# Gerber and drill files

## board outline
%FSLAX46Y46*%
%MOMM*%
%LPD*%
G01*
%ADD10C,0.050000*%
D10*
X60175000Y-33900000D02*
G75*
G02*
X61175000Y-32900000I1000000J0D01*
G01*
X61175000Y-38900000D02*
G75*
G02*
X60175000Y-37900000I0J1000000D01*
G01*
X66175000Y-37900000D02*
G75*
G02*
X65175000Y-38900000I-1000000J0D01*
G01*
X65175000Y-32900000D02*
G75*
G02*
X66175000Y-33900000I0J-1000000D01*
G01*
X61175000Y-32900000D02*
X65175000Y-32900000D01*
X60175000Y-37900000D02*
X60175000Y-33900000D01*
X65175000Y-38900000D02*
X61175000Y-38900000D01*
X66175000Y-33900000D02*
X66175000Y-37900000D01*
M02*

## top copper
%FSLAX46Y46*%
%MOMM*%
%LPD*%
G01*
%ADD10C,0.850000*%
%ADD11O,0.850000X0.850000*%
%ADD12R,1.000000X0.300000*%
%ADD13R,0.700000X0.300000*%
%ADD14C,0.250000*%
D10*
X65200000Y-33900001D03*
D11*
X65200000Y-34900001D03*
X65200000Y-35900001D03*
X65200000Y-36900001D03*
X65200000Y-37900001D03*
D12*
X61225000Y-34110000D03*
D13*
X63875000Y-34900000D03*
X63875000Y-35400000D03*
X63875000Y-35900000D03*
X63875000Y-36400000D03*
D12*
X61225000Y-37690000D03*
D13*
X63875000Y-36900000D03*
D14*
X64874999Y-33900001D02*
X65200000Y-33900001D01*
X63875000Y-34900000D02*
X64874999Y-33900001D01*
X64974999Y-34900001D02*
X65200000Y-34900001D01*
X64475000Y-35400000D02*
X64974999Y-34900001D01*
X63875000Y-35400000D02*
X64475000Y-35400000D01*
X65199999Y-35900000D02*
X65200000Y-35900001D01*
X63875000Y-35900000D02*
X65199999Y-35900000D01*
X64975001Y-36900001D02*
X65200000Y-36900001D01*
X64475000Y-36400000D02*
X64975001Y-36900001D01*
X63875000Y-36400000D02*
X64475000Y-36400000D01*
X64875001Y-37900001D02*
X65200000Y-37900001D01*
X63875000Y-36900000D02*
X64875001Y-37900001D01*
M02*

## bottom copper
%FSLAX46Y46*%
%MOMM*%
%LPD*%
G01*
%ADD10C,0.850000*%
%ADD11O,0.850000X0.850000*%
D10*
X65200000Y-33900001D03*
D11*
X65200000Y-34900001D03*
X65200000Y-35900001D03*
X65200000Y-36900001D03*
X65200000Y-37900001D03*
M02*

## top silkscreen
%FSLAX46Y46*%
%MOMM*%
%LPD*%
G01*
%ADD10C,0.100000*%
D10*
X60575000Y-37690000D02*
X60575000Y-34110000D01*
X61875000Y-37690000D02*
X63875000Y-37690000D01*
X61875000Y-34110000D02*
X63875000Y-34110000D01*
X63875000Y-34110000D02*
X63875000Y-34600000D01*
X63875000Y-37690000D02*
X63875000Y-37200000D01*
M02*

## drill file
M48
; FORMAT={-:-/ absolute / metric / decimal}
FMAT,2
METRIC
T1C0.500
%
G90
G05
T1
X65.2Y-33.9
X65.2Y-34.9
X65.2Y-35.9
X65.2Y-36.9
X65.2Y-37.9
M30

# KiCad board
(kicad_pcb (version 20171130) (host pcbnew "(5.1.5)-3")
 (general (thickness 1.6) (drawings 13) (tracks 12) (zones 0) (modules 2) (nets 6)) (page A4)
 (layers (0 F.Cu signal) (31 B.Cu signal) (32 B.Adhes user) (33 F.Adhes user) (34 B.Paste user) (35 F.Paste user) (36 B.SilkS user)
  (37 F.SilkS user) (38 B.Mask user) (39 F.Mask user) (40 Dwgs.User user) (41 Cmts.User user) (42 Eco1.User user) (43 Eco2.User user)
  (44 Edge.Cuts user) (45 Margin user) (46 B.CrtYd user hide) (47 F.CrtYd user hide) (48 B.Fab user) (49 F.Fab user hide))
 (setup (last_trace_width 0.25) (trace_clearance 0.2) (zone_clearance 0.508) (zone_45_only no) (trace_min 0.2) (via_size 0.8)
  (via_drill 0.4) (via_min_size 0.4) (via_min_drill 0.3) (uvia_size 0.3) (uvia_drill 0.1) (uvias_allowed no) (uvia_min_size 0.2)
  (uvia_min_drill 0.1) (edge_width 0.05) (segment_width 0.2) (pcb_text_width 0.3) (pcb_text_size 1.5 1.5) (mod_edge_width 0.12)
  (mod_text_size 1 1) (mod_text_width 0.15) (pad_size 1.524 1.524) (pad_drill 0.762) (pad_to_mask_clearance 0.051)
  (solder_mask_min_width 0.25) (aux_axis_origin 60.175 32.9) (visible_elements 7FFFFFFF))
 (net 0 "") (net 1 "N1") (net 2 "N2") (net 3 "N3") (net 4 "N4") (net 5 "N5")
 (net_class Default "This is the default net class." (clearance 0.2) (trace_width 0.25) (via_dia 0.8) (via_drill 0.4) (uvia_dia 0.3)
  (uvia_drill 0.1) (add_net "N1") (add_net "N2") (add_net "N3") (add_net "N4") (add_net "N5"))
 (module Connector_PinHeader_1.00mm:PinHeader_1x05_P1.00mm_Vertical (layer F.Cu) (at 65.2 33.900001)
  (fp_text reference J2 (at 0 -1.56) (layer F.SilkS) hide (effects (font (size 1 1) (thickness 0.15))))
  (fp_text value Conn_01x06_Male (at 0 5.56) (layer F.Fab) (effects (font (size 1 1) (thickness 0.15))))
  (pad 1 thru_hole circle (at 0 0) (size 0.85 0.85) (drill 0.5) (layers *.Cu *.Mask) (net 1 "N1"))
  (pad 2 thru_hole oval (at 0 1) (size 0.85 0.85) (drill 0.5) (layers *.Cu *.Mask) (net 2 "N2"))
  (pad 3 thru_hole oval (at 0 2) (size 0.85 0.85) (drill 0.5) (layers *.Cu *.Mask) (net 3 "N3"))
  (pad 4 thru_hole oval (at 0 3) (size 0.85 0.85) (drill 0.5) (layers *.Cu *.Mask) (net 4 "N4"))
  (pad 5 thru_hole oval (at 0 4) (size 0.85 0.85) (drill 0.5) (layers *.Cu *.Mask) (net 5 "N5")))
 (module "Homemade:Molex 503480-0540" (layer F.Cu) (at 62.425 35.9 270)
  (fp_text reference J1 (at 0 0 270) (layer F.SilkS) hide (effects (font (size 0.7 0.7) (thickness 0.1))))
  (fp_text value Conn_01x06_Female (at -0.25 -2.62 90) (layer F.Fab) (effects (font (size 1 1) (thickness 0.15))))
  (fp_line (start 1.79 1.85) (end -1.79 1.85) (layer F.SilkS) (width 0.1))
  (fp_line (start 1.79 0.55) (end 1.79 -1.45) (layer F.SilkS) (width 0.1))
  (fp_line (start -1.79 0.55) (end -1.79 -1.45) (layer F.SilkS) (width 0.1))
  (fp_line (start -1.79 -1.45) (end -1.3 -1.45) (layer F.SilkS) (width 0.1))
  (fp_line (start 1.79 -1.45) (end 1.3 -1.45) (layer F.SilkS) (width 0.1))
  (pad 6 smd rect (at -1.79 1.2 270) (size 0.3 1) (layers F.Cu F.Paste F.Mask))
  (pad 1 smd rect (at -1 -1.45 270) (size 0.3 0.7) (layers F.Cu F.Paste F.Mask) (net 1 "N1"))
  (pad 2 smd rect (at -0.5 -1.45 270) (size 0.3 0.7) (layers F.Cu F.Paste F.Mask) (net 2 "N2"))
  (pad 3 smd rect (at 0 -1.45 270) (size 0.3 0.7) (layers F.Cu F.Paste F.Mask) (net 3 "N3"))
  (pad 4 smd rect (at 0.5 -1.45 270) (size 0.3 0.7) (layers F.Cu F.Paste F.Mask) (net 4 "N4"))
  (pad 7 smd rect (at 1.79 1.2 270) (size 0.3 1) (layers F.Cu F.Paste F.Mask))
  (pad 5 smd rect (at 1 -1.45 270) (size 0.3 0.7) (layers F.Cu F.Paste F.Mask) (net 5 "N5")))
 (gr_arc (start 61.175 33.9) (end 61.175 32.9) (angle -90) (layer Edge.Cuts) (width 0.05))
 (gr_arc (start 61.175 37.9) (end 60.175 37.9) (angle -90) (layer Edge.Cuts) (width 0.05))
 (gr_arc (start 65.175 37.9) (end 65.175 38.9) (angle -90) (layer Edge.Cuts) (width 0.05))
 (gr_arc (start 65.175 33.9) (end 66.175 33.9) (angle -90) (layer Edge.Cuts) (width 0.05))
 (gr_line (start 61.175 32.9) (end 65.175 32.9) (layer Edge.Cuts) (width 0.05))
 (gr_line (start 60.175 37.9) (end 60.175 33.9) (layer Edge.Cuts) (width 0.05))
 (gr_line (start 65.175 38.9) (end 61.175 38.9) (layer Edge.Cuts) (width 0.05))
 (gr_line (start 66.175 33.9) (end 66.175 37.9) (layer Edge.Cuts) (width 0.05))
 (segment (start 64.874999 33.900001) (end 65.2 33.900001) (width 0.25) (layer F.Cu) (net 1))
 (segment (start 63.875 34.9) (end 64.874999 33.900001) (width 0.25) (layer F.Cu) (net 1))
 (segment (start 64.974999 34.900001) (end 65.2 34.900001) (width 0.25) (layer F.Cu) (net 2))
 (segment (start 64.475 35.4) (end 64.974999 34.900001) (width 0.25) (layer F.Cu) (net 2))
 (segment (start 63.875 35.4) (end 64.475 35.4) (width 0.25) (layer F.Cu) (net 2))
 (segment (start 65.199999 35.9) (end 65.2 35.900001) (width 0.25) (layer F.Cu) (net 3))
 (segment (start 63.875 35.9) (end 65.199999 35.9) (width 0.25) (layer F.Cu) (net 3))
 (segment (start 64.975001 36.900001) (end 65.2 36.900001) (width 0.25) (layer F.Cu) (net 4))
 (segment (start 64.475 36.4) (end 64.975001 36.900001) (width 0.25) (layer F.Cu) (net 4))
 (segment (start 63.875 36.4) (end 64.475 36.4) (width 0.25) (layer F.Cu) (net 4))
 (segment (start 64.875001 37.900001) (end 65.2 37.900001) (width 0.25) (layer F.Cu) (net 5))
 (segment (start 63.875 36.9) (end 64.875001 37.900001) (width 0.25) (layer F.Cu) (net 5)))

